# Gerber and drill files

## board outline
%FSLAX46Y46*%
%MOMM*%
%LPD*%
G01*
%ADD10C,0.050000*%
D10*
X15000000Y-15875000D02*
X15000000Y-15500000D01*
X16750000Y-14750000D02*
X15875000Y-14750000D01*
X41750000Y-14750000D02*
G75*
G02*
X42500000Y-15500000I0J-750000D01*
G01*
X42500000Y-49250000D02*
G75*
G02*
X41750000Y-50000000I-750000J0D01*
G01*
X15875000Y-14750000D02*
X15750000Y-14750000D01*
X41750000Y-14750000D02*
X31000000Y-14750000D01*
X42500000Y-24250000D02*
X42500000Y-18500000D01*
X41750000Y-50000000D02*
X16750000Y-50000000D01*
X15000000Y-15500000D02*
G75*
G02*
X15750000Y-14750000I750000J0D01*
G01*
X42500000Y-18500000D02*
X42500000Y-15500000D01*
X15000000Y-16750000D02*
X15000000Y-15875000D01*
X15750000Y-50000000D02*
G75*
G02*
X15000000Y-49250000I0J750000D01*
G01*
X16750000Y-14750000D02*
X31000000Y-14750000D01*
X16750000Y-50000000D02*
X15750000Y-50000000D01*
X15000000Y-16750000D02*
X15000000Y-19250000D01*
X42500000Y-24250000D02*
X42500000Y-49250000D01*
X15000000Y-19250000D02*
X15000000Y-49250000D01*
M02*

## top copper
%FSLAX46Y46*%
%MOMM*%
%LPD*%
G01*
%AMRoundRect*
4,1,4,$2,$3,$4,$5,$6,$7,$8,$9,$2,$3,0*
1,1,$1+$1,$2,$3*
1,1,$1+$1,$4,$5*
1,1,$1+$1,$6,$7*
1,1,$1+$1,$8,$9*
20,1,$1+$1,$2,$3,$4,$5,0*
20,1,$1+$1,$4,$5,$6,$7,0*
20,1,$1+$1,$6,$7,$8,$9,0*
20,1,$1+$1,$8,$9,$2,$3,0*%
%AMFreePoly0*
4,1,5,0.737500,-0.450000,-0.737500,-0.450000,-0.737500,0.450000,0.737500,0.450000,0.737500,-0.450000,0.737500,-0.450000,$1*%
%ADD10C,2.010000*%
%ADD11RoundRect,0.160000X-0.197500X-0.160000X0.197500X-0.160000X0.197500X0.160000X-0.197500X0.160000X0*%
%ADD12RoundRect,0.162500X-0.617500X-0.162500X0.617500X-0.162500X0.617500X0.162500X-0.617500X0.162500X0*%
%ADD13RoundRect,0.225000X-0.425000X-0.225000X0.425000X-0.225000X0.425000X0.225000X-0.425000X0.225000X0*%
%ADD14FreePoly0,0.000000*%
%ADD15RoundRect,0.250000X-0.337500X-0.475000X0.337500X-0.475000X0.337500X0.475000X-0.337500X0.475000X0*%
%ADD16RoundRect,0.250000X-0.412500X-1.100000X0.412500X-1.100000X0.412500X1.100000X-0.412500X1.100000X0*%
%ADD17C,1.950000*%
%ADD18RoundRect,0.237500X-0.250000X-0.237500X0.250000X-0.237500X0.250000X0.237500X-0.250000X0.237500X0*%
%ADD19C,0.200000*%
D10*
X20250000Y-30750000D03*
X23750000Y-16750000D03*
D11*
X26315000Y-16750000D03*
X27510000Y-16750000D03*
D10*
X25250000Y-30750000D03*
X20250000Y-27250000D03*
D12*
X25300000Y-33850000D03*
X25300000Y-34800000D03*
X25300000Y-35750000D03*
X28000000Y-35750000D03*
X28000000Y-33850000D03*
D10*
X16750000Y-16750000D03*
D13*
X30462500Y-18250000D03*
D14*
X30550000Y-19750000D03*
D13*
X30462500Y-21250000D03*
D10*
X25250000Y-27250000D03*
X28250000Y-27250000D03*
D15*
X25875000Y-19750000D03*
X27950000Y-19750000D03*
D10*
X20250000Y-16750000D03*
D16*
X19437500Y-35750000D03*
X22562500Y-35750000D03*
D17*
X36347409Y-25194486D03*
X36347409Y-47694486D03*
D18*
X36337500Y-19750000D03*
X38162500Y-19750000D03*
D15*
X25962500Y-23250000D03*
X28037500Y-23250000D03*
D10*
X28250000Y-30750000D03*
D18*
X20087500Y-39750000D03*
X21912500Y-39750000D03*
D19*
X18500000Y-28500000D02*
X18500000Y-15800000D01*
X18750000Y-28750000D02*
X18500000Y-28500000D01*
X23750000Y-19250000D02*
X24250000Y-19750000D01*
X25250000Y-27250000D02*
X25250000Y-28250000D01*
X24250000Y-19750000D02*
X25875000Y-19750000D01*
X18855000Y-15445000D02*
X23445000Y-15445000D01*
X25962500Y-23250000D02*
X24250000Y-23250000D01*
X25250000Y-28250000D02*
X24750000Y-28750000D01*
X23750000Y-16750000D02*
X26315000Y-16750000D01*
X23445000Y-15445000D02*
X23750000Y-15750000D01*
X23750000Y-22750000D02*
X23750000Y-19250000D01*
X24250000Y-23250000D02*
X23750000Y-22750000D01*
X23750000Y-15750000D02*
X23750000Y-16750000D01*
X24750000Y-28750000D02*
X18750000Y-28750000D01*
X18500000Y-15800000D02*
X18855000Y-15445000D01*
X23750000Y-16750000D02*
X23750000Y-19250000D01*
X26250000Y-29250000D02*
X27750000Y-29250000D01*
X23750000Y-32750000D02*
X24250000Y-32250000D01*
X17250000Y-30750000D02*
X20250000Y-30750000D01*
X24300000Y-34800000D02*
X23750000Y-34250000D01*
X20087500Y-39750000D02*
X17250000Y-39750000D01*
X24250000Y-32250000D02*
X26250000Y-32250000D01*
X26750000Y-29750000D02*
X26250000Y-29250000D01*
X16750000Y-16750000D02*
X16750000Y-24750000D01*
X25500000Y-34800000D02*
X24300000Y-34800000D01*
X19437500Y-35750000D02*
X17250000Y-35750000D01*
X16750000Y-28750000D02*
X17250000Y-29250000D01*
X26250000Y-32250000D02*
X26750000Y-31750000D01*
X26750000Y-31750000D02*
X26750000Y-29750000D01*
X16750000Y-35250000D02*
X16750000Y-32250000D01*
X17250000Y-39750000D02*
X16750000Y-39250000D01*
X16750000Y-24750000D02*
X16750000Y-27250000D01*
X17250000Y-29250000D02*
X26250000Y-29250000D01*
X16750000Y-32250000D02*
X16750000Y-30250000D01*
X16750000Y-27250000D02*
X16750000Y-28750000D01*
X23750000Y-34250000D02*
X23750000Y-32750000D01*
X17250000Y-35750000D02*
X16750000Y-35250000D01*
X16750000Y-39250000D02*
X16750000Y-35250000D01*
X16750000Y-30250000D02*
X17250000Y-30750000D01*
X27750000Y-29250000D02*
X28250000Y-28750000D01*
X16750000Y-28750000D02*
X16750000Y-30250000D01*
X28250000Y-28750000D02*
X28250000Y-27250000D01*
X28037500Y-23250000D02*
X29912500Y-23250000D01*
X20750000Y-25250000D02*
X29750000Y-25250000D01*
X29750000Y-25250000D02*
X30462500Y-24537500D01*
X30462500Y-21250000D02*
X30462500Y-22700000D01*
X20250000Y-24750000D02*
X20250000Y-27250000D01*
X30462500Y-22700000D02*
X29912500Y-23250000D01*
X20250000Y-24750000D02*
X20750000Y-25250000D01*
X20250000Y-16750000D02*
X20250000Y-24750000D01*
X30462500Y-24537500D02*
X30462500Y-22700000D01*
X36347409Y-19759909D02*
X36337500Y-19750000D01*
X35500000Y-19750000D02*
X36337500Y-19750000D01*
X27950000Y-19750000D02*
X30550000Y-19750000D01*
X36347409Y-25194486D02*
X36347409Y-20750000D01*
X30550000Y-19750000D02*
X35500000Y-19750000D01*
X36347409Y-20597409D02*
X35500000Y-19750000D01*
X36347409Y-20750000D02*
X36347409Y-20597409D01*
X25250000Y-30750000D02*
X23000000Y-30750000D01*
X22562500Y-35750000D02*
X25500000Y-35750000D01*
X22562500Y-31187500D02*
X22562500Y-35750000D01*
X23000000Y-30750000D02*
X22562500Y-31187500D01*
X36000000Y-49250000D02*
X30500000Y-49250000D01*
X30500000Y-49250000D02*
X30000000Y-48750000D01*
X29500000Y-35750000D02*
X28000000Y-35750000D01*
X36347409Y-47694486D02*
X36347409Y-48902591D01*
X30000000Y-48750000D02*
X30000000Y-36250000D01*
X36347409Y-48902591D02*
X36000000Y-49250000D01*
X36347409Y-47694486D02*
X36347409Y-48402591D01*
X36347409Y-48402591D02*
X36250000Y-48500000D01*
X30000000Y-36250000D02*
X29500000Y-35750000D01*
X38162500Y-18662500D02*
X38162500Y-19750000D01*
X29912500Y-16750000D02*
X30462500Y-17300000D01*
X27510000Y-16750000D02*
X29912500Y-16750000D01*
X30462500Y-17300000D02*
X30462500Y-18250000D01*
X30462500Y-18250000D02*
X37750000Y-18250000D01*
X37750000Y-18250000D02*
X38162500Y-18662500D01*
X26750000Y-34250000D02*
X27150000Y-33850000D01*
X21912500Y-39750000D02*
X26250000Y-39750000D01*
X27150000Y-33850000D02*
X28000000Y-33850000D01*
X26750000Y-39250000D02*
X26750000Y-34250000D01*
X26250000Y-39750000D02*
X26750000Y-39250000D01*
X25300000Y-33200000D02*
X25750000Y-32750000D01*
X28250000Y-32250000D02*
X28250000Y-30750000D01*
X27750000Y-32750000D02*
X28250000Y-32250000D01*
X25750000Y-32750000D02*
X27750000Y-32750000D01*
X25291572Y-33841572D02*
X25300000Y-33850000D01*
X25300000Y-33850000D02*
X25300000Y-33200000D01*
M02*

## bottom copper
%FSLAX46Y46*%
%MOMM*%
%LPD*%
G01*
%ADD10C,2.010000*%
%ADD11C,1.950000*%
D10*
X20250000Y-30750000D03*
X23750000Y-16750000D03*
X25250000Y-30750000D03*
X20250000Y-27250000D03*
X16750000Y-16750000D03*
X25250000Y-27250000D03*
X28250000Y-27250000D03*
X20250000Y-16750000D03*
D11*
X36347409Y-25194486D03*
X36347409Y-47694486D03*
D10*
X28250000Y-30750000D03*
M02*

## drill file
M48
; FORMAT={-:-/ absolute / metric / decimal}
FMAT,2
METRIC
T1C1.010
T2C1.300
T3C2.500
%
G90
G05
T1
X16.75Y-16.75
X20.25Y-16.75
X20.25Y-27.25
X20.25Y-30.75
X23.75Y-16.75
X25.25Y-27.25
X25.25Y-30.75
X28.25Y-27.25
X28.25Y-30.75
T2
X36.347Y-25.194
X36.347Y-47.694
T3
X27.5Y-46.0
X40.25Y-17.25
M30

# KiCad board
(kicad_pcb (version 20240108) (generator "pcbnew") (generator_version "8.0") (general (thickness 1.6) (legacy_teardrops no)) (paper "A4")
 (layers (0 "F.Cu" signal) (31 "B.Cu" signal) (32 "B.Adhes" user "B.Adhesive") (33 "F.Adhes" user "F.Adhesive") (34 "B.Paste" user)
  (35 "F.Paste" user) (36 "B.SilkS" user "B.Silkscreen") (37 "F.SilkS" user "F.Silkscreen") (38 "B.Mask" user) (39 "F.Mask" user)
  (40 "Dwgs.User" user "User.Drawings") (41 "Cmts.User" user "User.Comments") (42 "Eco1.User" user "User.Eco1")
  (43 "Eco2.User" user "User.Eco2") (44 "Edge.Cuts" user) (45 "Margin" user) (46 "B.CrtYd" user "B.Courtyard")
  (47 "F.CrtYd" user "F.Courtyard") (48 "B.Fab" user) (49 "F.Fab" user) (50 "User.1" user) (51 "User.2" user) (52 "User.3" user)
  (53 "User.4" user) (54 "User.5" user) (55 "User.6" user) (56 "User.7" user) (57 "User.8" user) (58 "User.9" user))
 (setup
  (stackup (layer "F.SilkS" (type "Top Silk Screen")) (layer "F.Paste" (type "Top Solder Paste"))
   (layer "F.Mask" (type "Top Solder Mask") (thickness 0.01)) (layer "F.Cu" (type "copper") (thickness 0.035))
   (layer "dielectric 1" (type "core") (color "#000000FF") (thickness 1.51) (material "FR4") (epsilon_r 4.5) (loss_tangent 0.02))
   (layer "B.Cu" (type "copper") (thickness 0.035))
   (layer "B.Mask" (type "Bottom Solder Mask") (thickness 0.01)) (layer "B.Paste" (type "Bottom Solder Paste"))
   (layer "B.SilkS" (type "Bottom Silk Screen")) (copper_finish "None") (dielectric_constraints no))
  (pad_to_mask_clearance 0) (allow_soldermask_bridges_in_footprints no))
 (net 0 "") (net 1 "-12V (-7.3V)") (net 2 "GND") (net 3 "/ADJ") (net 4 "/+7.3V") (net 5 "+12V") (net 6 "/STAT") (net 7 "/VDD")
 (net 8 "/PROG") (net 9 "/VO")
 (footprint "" (layer "F.Cu") (at 20.25 30.75)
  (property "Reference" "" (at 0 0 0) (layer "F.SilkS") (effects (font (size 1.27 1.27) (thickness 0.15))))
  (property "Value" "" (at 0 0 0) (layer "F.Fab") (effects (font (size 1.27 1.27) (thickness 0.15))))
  (pad "-12V FAN" thru_hole circle (at 0 0) (size 2.01 2.01) (drill 1.01) (layers "*.Cu" "*.Mask") (remove_unused_layers no)
   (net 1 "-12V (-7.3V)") (thermal_bridge_angle 0)))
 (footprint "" (layer "F.Cu") (at 27.5 46)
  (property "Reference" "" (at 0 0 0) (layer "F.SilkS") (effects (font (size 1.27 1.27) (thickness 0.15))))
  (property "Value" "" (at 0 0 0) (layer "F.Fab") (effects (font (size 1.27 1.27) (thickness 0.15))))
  (pad "" np_thru_hole circle (at 0 0) (size 2.5 2.5) (drill 2.5) (layers "F&B.Cu" "*.Mask") (thermal_bridge_angle 0)))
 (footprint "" (layer "F.Cu") (at 23.75 16.75)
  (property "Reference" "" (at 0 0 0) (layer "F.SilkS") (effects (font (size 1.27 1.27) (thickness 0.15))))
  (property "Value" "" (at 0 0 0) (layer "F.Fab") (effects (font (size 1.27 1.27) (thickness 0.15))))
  (pad "GND" thru_hole circle (at 0 0) (size 2.01 2.01) (drill 1.01) (layers "*.Cu" "*.Mask") (remove_unused_layers no) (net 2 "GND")
   (thermal_bridge_angle 0)))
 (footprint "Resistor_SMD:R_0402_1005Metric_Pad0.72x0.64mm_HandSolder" (layer "F.Cu") (at 26.9125 16.75)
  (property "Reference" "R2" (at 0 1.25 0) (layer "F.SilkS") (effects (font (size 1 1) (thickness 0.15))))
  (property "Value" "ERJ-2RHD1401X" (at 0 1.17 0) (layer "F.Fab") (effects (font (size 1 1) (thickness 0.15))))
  (pad "1" smd roundrect (at -0.5975 0) (size 0.715 0.64) (layers "F.Cu" "F.Paste" "F.Mask") (roundrect_rratio 0.25) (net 2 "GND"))
  (pad "2" smd roundrect (at 0.5975 0) (size 0.715 0.64) (layers "F.Cu" "F.Paste" "F.Mask") (roundrect_rratio 0.25) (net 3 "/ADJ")))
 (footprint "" (layer "F.Cu") (at 25.25 30.75)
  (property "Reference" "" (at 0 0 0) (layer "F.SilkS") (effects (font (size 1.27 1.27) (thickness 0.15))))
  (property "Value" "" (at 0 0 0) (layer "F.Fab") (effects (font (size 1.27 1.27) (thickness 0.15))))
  (pad "-12V FAN" thru_hole circle (at 0 0) (size 2.01 2.01) (drill 1.01) (layers "*.Cu" "*.Mask") (remove_unused_layers no)
   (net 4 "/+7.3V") (thermal_bridge_angle 0)))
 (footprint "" (layer "F.Cu") (at 20.25 27.25)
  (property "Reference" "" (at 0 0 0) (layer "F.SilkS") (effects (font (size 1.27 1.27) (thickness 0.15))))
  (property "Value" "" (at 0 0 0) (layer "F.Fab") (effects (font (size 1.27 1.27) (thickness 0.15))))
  (pad "+12V FAN" thru_hole circle (at 0 0) (size 2.01 2.01) (drill 1.01) (layers "*.Cu" "*.Mask") (remove_unused_layers no) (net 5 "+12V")
   (thermal_bridge_angle 0)))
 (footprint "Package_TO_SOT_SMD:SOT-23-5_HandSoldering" (layer "F.Cu") (at 26.65 34.8)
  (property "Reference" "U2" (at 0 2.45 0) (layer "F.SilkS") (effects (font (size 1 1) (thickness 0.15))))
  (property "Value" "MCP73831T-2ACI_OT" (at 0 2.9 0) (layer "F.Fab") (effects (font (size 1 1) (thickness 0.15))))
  (pad "1" smd roundrect (at -1.35 -0.95) (size 1.56 0.65) (layers "F.Cu" "F.Paste" "F.Mask") (roundrect_rratio 0.25) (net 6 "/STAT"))
  (pad "2" smd roundrect (at -1.35 0) (size 1.56 0.65) (layers "F.Cu" "F.Paste" "F.Mask") (roundrect_rratio 0.25) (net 1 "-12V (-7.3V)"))
  (pad "3" smd roundrect (at -1.35 0.95) (size 1.56 0.65) (layers "F.Cu" "F.Paste" "F.Mask") (roundrect_rratio 0.25) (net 4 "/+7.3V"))
  (pad "4" smd roundrect (at 1.35 0.95) (size 1.56 0.65) (layers "F.Cu" "F.Paste" "F.Mask") (roundrect_rratio 0.25) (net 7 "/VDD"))
  (pad "5" smd roundrect (at 1.35 -0.95) (size 1.56 0.65) (layers "F.Cu" "F.Paste" "F.Mask") (roundrect_rratio 0.25) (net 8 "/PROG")))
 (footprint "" (layer "F.Cu") (at 16.75 16.75)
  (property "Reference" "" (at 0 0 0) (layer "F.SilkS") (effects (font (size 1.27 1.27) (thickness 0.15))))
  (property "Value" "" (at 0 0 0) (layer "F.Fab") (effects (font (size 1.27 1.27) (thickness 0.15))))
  (pad "-12V" thru_hole circle (at 0 0) (size 2.01 2.01) (drill 1.01) (layers "*.Cu" "*.Mask") (remove_unused_layers no)
   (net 1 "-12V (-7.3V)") (thermal_bridge_angle 0)))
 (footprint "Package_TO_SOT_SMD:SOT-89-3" (layer "F.Cu") (at 32.4125 19.75)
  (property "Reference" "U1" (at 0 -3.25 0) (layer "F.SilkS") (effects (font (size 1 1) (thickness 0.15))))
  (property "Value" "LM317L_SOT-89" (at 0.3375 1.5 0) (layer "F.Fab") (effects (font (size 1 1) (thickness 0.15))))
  (pad "1" smd roundrect (at -1.95 -1.5) (size 1.3 0.9) (layers "F.Cu" "F.Paste" "F.Mask") (roundrect_rratio 0.25) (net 3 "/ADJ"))
  (pad "2" smd custom (at -1.8625 0) (size 1.475 0.9) (layers "F.Cu" "F.Paste" "F.Mask") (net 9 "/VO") (zone_connect 2)
   (thermal_bridge_angle 45) (options (clearance outline) (anchor rect)) (primitives))
  (pad "3" smd roundrect (at -1.95 1.5) (size 1.3 0.9) (layers "F.Cu" "F.Paste" "F.Mask") (roundrect_rratio 0.25) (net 5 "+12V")))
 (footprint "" (layer "F.Cu") (at 25.25 27.25)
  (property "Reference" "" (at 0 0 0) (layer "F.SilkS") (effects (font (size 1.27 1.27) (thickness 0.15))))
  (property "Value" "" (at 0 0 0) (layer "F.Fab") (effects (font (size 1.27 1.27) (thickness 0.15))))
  (pad "-12V FAN" thru_hole circle (at 0 0) (size 2.01 2.01) (drill 1.01) (layers "*.Cu" "*.Mask") (remove_unused_layers no) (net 2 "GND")
   (thermal_bridge_angle 0)))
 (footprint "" (layer "F.Cu") (at 28.25 27.25)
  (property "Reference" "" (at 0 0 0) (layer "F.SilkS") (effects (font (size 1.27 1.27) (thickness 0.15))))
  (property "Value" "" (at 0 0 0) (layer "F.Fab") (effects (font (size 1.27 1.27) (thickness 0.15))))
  (pad "-12V FAN" thru_hole circle (at 0 0) (size 2.01 2.01) (drill 1.01) (layers "*.Cu" "*.Mask") (remove_unused_layers no)
   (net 1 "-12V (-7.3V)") (thermal_bridge_angle 0)))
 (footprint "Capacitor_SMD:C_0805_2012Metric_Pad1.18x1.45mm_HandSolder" (layer "F.Cu") (at 26.9125 19.75)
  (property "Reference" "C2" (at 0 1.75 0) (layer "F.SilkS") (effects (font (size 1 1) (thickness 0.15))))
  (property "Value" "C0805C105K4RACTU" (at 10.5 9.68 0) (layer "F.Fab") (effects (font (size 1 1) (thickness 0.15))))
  (pad "1" smd roundrect (at -1.0375 0) (size 1.175 1.45) (layers "F.Cu" "F.Paste" "F.Mask") (roundrect_rratio 0.212766) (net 2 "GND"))
  (pad "2" smd roundrect (at 1.0375 0) (size 1.175 1.45) (layers "F.Cu" "F.Paste" "F.Mask") (roundrect_rratio 0.212766) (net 9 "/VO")))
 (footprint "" (layer "F.Cu") (at 20.25 16.75)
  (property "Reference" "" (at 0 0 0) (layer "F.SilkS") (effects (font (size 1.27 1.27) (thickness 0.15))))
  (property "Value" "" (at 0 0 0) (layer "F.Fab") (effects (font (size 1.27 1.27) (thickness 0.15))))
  (pad "+12V" thru_hole circle (at 0 0) (size 2.01 2.01) (drill 1.01) (layers "*.Cu" "*.Mask") (remove_unused_layers no) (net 5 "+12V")
   (thermal_bridge_angle 0)))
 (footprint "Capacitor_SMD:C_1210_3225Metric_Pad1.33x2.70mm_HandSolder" (layer "F.Cu") (at 21 35.75)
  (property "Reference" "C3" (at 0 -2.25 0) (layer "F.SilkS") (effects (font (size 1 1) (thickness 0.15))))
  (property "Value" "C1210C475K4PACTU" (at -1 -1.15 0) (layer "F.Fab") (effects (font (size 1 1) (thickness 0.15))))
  (pad "1" smd roundrect (at -1.5625 0) (size 1.325 2.7) (layers "F.Cu" "F.Paste" "F.Mask") (roundrect_rratio 0.188679)
   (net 1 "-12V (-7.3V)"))
  (pad "2" smd roundrect (at 1.5625 0) (size 1.325 2.7) (layers "F.Cu" "F.Paste" "F.Mask") (roundrect_rratio 0.188679) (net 4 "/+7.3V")))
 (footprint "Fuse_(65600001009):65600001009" (layer "F.Cu") (at 36.347409 36.444486 -90)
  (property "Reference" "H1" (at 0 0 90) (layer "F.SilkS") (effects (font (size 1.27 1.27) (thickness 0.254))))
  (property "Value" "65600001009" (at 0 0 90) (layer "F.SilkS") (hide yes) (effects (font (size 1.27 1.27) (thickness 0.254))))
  (pad "1" thru_hole circle (at -11.25 0 270) (size 1.95 1.95) (drill 1.3) (layers "*.Cu" "*.Mask") (remove_unused_layers no) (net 9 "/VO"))
  (pad "2" thru_hole circle (at 11.25 0 270) (size 1.95 1.95) (drill 1.3) (layers "*.Cu" "*.Mask") (remove_unused_layers no) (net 7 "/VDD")))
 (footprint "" (layer "F.Cu") (at 40.25 17.25)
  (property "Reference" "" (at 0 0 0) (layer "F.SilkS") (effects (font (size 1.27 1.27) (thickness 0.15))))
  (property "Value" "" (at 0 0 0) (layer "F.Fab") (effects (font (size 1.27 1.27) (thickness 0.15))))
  (pad "" np_thru_hole circle (at 0 0) (size 2.5 2.5) (drill 2.5) (layers "F&B.Cu" "*.Mask") (thermal_bridge_angle 0)))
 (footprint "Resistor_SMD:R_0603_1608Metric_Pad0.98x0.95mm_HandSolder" (layer "F.Cu") (at 37.25 19.75)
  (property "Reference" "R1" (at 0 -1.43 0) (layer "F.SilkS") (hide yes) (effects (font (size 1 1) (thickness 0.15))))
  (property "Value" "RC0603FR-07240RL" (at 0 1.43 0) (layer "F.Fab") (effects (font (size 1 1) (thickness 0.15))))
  (pad "1" smd roundrect (at -0.9125 0) (size 0.975 0.95) (layers "F.Cu" "F.Paste" "F.Mask") (roundrect_rratio 0.25) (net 9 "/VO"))
  (pad "2" smd roundrect (at 0.9125 0) (size 0.975 0.95) (layers "F.Cu" "F.Paste" "F.Mask") (roundrect_rratio 0.25) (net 3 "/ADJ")))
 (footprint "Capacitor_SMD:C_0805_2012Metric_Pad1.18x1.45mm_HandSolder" (layer "F.Cu") (at 27 23.25)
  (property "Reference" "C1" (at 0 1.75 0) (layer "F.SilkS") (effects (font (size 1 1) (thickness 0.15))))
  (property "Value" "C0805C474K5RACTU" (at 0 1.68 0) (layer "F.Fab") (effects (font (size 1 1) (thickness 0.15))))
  (pad "1" smd roundrect (at -1.0375 0) (size 1.175 1.45) (layers "F.Cu" "F.Paste" "F.Mask") (roundrect_rratio 0.212766) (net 2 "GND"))
  (pad "2" smd roundrect (at 1.0375 0) (size 1.175 1.45) (layers "F.Cu" "F.Paste" "F.Mask") (roundrect_rratio 0.212766) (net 5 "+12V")))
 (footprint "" (layer "F.Cu") (at 28.25 30.75 90)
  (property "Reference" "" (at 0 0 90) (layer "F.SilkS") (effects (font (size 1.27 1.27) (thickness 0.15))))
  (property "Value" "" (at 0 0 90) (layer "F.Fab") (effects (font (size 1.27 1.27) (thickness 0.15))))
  (pad "STAT" thru_hole circle (at 0 0 90) (size 2.01 2.01) (drill 1.01) (layers "*.Cu" "*.Mask") (remove_unused_layers no) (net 6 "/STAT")
   (thermal_bridge_angle 0)))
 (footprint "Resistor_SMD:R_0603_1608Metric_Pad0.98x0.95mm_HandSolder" (layer "F.Cu") (at 21 39.75)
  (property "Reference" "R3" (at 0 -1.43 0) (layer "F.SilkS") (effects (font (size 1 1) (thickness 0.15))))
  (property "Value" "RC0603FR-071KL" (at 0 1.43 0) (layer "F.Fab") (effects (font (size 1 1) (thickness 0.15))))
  (pad "1" smd roundrect (at -0.9125 0) (size 0.975 0.95) (layers "F.Cu" "F.Paste" "F.Mask") (roundrect_rratio 0.25) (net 1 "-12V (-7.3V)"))
  (pad "2" smd roundrect (at 0.9125 0) (size 0.975 0.95) (layers "F.Cu" "F.Paste" "F.Mask") (roundrect_rratio 0.25) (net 8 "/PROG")))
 (gr_line (start 15 15.875) (end 15 15.5) (stroke (width 0.05) (type default)) (layer "Edge.Cuts"))
 (gr_line (start 16.75 14.75) (end 15.875 14.75) (stroke (width 0.05) (type default)) (layer "Edge.Cuts"))
 (gr_arc (start 41.75 14.75) (mid 42.28033 14.96967) (end 42.5 15.5) (stroke (width 0.05) (type default)) (layer "Edge.Cuts"))
 (gr_arc (start 42.5 49.25) (mid 42.28033 49.78033) (end 41.75 50) (stroke (width 0.05) (type default)) (layer "Edge.Cuts"))
 (gr_line (start 15.875 14.75) (end 15.75 14.75) (stroke (width 0.05) (type default)) (layer "Edge.Cuts"))
 (gr_line (start 41.75 14.75) (end 31 14.75) (stroke (width 0.05) (type default)) (layer "Edge.Cuts"))
 (gr_line (start 42.5 24.25) (end 42.5 18.5) (stroke (width 0.05) (type default)) (layer "Edge.Cuts"))
 (gr_line (start 41.75 50) (end 16.75 50) (stroke (width 0.05) (type default)) (layer "Edge.Cuts"))
 (gr_arc (start 15 15.5) (mid 15.21967 14.96967) (end 15.75 14.75) (stroke (width 0.05) (type default)) (layer "Edge.Cuts"))
 (gr_line (start 42.5 18.5) (end 42.5 15.5) (stroke (width 0.05) (type default)) (layer "Edge.Cuts"))
 (gr_line (start 15 16.75) (end 15 15.875) (stroke (width 0.05) (type default)) (layer "Edge.Cuts"))
 (gr_arc (start 15.75 50) (mid 15.21967 49.78033) (end 15 49.25) (stroke (width 0.05) (type default)) (layer "Edge.Cuts"))
 (gr_line (start 16.75 14.75) (end 31 14.75) (stroke (width 0.05) (type default)) (layer "Edge.Cuts"))
 (gr_line (start 16.75 50) (end 15.75 50) (stroke (width 0.05) (type default)) (layer "Edge.Cuts"))
 (gr_line (start 15 16.75) (end 15 19.25) (stroke (width 0.05) (type default)) (layer "Edge.Cuts"))
 (gr_line (start 42.5 24.25) (end 42.5 49.25) (stroke (width 0.05) (type default)) (layer "Edge.Cuts"))
 (gr_line (start 15 19.25) (end 15 49.25) (stroke (width 0.05) (type default)) (layer "Edge.Cuts"))
 (segment (start 18.5 28.5) (end 18.5 15.8) (width 0.2) (layer "F.Cu") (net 2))
 (segment (start 18.75 28.75) (end 18.5 28.5) (width 0.2) (layer "F.Cu") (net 2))
 (segment (start 23.75 19.25) (end 24.25 19.75) (width 0.2) (layer "F.Cu") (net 2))
 (segment (start 25.25 27.25) (end 25.25 28.25) (width 0.2) (layer "F.Cu") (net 2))
 (segment (start 24.25 19.75) (end 25.875 19.75) (width 0.2) (layer "F.Cu") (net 2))
 (segment (start 18.855 15.445) (end 23.445 15.445) (width 0.2) (layer "F.Cu") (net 2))
 (segment (start 25.9625 23.25) (end 24.25 23.25) (width 0.2) (layer "F.Cu") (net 2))
 (segment (start 25.25 28.25) (end 24.75 28.75) (width 0.2) (layer "F.Cu") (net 2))
 (segment (start 23.75 16.75) (end 26.315 16.75) (width 0.2) (layer "F.Cu") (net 2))
 (segment (start 23.445 15.445) (end 23.75 15.75) (width 0.2) (layer "F.Cu") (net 2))
 (segment (start 23.75 22.75) (end 23.75 19.25) (width 0.2) (layer "F.Cu") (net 2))
 (segment (start 24.25 23.25) (end 23.75 22.75) (width 0.2) (layer "F.Cu") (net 2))
 (segment (start 23.75 15.75) (end 23.75 16.75) (width 0.2) (layer "F.Cu") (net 2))
 (segment (start 24.75 28.75) (end 18.75 28.75) (width 0.2) (layer "F.Cu") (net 2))
 (segment (start 18.5 15.8) (end 18.855 15.445) (width 0.2) (layer "F.Cu") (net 2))
 (segment (start 23.75 16.75) (end 23.75 19.25) (width 0.2) (layer "F.Cu") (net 2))
 (segment (start 26.25 29.25) (end 27.75 29.25) (width 0.2) (layer "F.Cu") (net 1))
 (segment (start 23.75 32.75) (end 24.25 32.25) (width 0.2) (layer "F.Cu") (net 1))
 (segment (start 17.25 30.75) (end 20.25 30.75) (width 0.2) (layer "F.Cu") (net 1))
 (segment (start 24.3 34.8) (end 23.75 34.25) (width 0.2) (layer "F.Cu") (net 1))
 (segment (start 20.0875 39.75) (end 17.25 39.75) (width 0.2) (layer "F.Cu") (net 1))
 (segment (start 24.25 32.25) (end 26.25 32.25) (width 0.2) (layer "F.Cu") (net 1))
 (segment (start 26.75 29.75) (end 26.25 29.25) (width 0.2) (layer "F.Cu") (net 1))
 (segment (start 16.75 16.75) (end 16.75 24.75) (width 0.2) (layer "F.Cu") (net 1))
 (segment (start 25.5 34.8) (end 24.3 34.8) (width 0.2) (layer "F.Cu") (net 1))
 (segment (start 19.4375 35.75) (end 17.25 35.75) (width 0.2) (layer "F.Cu") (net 1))
 (segment (start 16.75 28.75) (end 17.25 29.25) (width 0.2) (layer "F.Cu") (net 1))
 (segment (start 26.25 32.25) (end 26.75 31.75) (width 0.2) (layer "F.Cu") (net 1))
 (segment (start 26.75 31.75) (end 26.75 29.75) (width 0.2) (layer "F.Cu") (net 1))
 (segment (start 16.75 35.25) (end 16.75 32.25) (width 0.2) (layer "F.Cu") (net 1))
 (segment (start 17.25 39.75) (end 16.75 39.25) (width 0.2) (layer "F.Cu") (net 1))
 (segment (start 16.75 24.75) (end 16.75 27.25) (width 0.2) (layer "F.Cu") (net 1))
 (segment (start 17.25 29.25) (end 26.25 29.25) (width 0.2) (layer "F.Cu") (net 1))
 (segment (start 16.75 32.25) (end 16.75 30.25) (width 0.2) (layer "F.Cu") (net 1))
 (segment (start 16.75 27.25) (end 16.75 28.75) (width 0.2) (layer "F.Cu") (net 1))
 (segment (start 23.75 34.25) (end 23.75 32.75) (width 0.2) (layer "F.Cu") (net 1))
 (segment (start 17.25 35.75) (end 16.75 35.25) (width 0.2) (layer "F.Cu") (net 1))
 (segment (start 16.75 39.25) (end 16.75 35.25) (width 0.2) (layer "F.Cu") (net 1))
 (segment (start 16.75 30.25) (end 17.25 30.75) (width 0.2) (layer "F.Cu") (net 1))
 (segment (start 27.75 29.25) (end 28.25 28.75) (width 0.2) (layer "F.Cu") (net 1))
 (segment (start 16.75 28.75) (end 16.75 30.25) (width 0.2) (layer "F.Cu") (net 1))
 (segment (start 28.25 28.75) (end 28.25 27.25) (width 0.2) (layer "F.Cu") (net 1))
 (segment (start 28.0375 23.25) (end 29.9125 23.25) (width 0.2) (layer "F.Cu") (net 5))
 (segment (start 20.75 25.25) (end 29.75 25.25) (width 0.2) (layer "F.Cu") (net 5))
 (segment (start 29.75 25.25) (end 30.4625 24.5375) (width 0.2) (layer "F.Cu") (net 5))
 (segment (start 30.4625 21.25) (end 30.4625 22.7) (width 0.2) (layer "F.Cu") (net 5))
 (segment (start 20.25 24.75) (end 20.25 27.25) (width 0.2) (layer "F.Cu") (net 5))
 (segment (start 30.4625 22.7) (end 29.9125 23.25) (width 0.2) (layer "F.Cu") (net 5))
 (segment (start 20.25 24.75) (end 20.75 25.25) (width 0.2) (layer "F.Cu") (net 5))
 (segment (start 20.25 16.75) (end 20.25 24.75) (width 0.2) (layer "F.Cu") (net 5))
 (segment (start 30.4625 24.5375) (end 30.4625 22.7) (width 0.2) (layer "F.Cu") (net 5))
 (segment (start 36.347409 19.759909) (end 36.3375 19.75) (width 0.2) (layer "F.Cu") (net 9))
 (segment (start 35.5 19.75) (end 36.3375 19.75) (width 0.2) (layer "F.Cu") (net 9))
 (segment (start 27.95 19.75) (end 30.55 19.75) (width 0.2) (layer "F.Cu") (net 9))
 (segment (start 36.347409 25.194486) (end 36.347409 20.75) (width 0.2) (layer "F.Cu") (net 9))
 (segment (start 30.55 19.75) (end 35.5 19.75) (width 0.2) (layer "F.Cu") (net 9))
 (segment (start 36.347409 20.597409) (end 35.5 19.75) (width 0.2) (layer "F.Cu") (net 9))
 (segment (start 36.347409 20.75) (end 36.347409 20.597409) (width 0.2) (layer "F.Cu") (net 9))
 (segment (start 25.25 30.75) (end 23 30.75) (width 0.2) (layer "F.Cu") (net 4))
 (segment (start 22.5625 35.75) (end 25.5 35.75) (width 0.2) (layer "F.Cu") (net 4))
 (segment (start 22.5625 31.1875) (end 22.5625 35.75) (width 0.2) (layer "F.Cu") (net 4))
 (segment (start 23 30.75) (end 22.5625 31.1875) (width 0.2) (layer "F.Cu") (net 4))
 (segment (start 36 49.25) (end 30.5 49.25) (width 0.2) (layer "F.Cu") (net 7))
 (segment (start 30.5 49.25) (end 30 48.75) (width 0.2) (layer "F.Cu") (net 7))
 (segment (start 29.5 35.75) (end 28 35.75) (width 0.2) (layer "F.Cu") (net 7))
 (segment (start 36.347409 47.694486) (end 36.347409 48.902591) (width 0.2) (layer "F.Cu") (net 7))
 (segment (start 30 48.75) (end 30 36.25) (width 0.2) (layer "F.Cu") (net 7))
 (segment (start 36.347409 48.902591) (end 36 49.25) (width 0.2) (layer "F.Cu") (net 7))
 (segment (start 36.347409 47.694486) (end 36.347409 48.402591) (width 0.2) (layer "F.Cu") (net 7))
 (segment (start 36.347409 48.402591) (end 36.25 48.5) (width 0.2) (layer "F.Cu") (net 7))
 (segment (start 30 36.25) (end 29.5 35.75) (width 0.2) (layer "F.Cu") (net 7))
 (segment (start 38.1625 18.6625) (end 38.1625 19.75) (width 0.2) (layer "F.Cu") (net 3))
 (segment (start 29.9125 16.75) (end 30.4625 17.3) (width 0.2) (layer "F.Cu") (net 3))
 (segment (start 27.51 16.75) (end 29.9125 16.75) (width 0.2) (layer "F.Cu") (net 3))
 (segment (start 30.4625 17.3) (end 30.4625 18.25) (width 0.2) (layer "F.Cu") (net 3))
 (segment (start 30.4625 18.25) (end 37.75 18.25) (width 0.2) (layer "F.Cu") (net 3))
 (segment (start 37.75 18.25) (end 38.1625 18.6625) (width 0.2) (layer "F.Cu") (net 3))
 (segment (start 26.75 34.25) (end 27.15 33.85) (width 0.2) (layer "F.Cu") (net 8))
 (segment (start 21.9125 39.75) (end 26.25 39.75) (width 0.2) (layer "F.Cu") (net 8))
 (segment (start 27.15 33.85) (end 28 33.85) (width 0.2) (layer "F.Cu") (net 8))
 (segment (start 26.75 39.25) (end 26.75 34.25) (width 0.2) (layer "F.Cu") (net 8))
 (segment (start 26.25 39.75) (end 26.75 39.25) (width 0.2) (layer "F.Cu") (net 8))
 (segment (start 25.3 33.2) (end 25.75 32.75) (width 0.2) (layer "F.Cu") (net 6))
 (segment (start 28.25 32.25) (end 28.25 30.75) (width 0.2) (layer "F.Cu") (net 6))
 (segment (start 27.75 32.75) (end 28.25 32.25) (width 0.2) (layer "F.Cu") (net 6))
 (segment (start 25.75 32.75) (end 27.75 32.75) (width 0.2) (layer "F.Cu") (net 6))
 (segment (start 25.291572 33.841572) (end 25.3 33.85) (width 0.2) (layer "F.Cu") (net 6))
 (segment (start 25.3 33.85) (end 25.3 33.2) (width 0.2) (layer "F.Cu") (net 6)))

